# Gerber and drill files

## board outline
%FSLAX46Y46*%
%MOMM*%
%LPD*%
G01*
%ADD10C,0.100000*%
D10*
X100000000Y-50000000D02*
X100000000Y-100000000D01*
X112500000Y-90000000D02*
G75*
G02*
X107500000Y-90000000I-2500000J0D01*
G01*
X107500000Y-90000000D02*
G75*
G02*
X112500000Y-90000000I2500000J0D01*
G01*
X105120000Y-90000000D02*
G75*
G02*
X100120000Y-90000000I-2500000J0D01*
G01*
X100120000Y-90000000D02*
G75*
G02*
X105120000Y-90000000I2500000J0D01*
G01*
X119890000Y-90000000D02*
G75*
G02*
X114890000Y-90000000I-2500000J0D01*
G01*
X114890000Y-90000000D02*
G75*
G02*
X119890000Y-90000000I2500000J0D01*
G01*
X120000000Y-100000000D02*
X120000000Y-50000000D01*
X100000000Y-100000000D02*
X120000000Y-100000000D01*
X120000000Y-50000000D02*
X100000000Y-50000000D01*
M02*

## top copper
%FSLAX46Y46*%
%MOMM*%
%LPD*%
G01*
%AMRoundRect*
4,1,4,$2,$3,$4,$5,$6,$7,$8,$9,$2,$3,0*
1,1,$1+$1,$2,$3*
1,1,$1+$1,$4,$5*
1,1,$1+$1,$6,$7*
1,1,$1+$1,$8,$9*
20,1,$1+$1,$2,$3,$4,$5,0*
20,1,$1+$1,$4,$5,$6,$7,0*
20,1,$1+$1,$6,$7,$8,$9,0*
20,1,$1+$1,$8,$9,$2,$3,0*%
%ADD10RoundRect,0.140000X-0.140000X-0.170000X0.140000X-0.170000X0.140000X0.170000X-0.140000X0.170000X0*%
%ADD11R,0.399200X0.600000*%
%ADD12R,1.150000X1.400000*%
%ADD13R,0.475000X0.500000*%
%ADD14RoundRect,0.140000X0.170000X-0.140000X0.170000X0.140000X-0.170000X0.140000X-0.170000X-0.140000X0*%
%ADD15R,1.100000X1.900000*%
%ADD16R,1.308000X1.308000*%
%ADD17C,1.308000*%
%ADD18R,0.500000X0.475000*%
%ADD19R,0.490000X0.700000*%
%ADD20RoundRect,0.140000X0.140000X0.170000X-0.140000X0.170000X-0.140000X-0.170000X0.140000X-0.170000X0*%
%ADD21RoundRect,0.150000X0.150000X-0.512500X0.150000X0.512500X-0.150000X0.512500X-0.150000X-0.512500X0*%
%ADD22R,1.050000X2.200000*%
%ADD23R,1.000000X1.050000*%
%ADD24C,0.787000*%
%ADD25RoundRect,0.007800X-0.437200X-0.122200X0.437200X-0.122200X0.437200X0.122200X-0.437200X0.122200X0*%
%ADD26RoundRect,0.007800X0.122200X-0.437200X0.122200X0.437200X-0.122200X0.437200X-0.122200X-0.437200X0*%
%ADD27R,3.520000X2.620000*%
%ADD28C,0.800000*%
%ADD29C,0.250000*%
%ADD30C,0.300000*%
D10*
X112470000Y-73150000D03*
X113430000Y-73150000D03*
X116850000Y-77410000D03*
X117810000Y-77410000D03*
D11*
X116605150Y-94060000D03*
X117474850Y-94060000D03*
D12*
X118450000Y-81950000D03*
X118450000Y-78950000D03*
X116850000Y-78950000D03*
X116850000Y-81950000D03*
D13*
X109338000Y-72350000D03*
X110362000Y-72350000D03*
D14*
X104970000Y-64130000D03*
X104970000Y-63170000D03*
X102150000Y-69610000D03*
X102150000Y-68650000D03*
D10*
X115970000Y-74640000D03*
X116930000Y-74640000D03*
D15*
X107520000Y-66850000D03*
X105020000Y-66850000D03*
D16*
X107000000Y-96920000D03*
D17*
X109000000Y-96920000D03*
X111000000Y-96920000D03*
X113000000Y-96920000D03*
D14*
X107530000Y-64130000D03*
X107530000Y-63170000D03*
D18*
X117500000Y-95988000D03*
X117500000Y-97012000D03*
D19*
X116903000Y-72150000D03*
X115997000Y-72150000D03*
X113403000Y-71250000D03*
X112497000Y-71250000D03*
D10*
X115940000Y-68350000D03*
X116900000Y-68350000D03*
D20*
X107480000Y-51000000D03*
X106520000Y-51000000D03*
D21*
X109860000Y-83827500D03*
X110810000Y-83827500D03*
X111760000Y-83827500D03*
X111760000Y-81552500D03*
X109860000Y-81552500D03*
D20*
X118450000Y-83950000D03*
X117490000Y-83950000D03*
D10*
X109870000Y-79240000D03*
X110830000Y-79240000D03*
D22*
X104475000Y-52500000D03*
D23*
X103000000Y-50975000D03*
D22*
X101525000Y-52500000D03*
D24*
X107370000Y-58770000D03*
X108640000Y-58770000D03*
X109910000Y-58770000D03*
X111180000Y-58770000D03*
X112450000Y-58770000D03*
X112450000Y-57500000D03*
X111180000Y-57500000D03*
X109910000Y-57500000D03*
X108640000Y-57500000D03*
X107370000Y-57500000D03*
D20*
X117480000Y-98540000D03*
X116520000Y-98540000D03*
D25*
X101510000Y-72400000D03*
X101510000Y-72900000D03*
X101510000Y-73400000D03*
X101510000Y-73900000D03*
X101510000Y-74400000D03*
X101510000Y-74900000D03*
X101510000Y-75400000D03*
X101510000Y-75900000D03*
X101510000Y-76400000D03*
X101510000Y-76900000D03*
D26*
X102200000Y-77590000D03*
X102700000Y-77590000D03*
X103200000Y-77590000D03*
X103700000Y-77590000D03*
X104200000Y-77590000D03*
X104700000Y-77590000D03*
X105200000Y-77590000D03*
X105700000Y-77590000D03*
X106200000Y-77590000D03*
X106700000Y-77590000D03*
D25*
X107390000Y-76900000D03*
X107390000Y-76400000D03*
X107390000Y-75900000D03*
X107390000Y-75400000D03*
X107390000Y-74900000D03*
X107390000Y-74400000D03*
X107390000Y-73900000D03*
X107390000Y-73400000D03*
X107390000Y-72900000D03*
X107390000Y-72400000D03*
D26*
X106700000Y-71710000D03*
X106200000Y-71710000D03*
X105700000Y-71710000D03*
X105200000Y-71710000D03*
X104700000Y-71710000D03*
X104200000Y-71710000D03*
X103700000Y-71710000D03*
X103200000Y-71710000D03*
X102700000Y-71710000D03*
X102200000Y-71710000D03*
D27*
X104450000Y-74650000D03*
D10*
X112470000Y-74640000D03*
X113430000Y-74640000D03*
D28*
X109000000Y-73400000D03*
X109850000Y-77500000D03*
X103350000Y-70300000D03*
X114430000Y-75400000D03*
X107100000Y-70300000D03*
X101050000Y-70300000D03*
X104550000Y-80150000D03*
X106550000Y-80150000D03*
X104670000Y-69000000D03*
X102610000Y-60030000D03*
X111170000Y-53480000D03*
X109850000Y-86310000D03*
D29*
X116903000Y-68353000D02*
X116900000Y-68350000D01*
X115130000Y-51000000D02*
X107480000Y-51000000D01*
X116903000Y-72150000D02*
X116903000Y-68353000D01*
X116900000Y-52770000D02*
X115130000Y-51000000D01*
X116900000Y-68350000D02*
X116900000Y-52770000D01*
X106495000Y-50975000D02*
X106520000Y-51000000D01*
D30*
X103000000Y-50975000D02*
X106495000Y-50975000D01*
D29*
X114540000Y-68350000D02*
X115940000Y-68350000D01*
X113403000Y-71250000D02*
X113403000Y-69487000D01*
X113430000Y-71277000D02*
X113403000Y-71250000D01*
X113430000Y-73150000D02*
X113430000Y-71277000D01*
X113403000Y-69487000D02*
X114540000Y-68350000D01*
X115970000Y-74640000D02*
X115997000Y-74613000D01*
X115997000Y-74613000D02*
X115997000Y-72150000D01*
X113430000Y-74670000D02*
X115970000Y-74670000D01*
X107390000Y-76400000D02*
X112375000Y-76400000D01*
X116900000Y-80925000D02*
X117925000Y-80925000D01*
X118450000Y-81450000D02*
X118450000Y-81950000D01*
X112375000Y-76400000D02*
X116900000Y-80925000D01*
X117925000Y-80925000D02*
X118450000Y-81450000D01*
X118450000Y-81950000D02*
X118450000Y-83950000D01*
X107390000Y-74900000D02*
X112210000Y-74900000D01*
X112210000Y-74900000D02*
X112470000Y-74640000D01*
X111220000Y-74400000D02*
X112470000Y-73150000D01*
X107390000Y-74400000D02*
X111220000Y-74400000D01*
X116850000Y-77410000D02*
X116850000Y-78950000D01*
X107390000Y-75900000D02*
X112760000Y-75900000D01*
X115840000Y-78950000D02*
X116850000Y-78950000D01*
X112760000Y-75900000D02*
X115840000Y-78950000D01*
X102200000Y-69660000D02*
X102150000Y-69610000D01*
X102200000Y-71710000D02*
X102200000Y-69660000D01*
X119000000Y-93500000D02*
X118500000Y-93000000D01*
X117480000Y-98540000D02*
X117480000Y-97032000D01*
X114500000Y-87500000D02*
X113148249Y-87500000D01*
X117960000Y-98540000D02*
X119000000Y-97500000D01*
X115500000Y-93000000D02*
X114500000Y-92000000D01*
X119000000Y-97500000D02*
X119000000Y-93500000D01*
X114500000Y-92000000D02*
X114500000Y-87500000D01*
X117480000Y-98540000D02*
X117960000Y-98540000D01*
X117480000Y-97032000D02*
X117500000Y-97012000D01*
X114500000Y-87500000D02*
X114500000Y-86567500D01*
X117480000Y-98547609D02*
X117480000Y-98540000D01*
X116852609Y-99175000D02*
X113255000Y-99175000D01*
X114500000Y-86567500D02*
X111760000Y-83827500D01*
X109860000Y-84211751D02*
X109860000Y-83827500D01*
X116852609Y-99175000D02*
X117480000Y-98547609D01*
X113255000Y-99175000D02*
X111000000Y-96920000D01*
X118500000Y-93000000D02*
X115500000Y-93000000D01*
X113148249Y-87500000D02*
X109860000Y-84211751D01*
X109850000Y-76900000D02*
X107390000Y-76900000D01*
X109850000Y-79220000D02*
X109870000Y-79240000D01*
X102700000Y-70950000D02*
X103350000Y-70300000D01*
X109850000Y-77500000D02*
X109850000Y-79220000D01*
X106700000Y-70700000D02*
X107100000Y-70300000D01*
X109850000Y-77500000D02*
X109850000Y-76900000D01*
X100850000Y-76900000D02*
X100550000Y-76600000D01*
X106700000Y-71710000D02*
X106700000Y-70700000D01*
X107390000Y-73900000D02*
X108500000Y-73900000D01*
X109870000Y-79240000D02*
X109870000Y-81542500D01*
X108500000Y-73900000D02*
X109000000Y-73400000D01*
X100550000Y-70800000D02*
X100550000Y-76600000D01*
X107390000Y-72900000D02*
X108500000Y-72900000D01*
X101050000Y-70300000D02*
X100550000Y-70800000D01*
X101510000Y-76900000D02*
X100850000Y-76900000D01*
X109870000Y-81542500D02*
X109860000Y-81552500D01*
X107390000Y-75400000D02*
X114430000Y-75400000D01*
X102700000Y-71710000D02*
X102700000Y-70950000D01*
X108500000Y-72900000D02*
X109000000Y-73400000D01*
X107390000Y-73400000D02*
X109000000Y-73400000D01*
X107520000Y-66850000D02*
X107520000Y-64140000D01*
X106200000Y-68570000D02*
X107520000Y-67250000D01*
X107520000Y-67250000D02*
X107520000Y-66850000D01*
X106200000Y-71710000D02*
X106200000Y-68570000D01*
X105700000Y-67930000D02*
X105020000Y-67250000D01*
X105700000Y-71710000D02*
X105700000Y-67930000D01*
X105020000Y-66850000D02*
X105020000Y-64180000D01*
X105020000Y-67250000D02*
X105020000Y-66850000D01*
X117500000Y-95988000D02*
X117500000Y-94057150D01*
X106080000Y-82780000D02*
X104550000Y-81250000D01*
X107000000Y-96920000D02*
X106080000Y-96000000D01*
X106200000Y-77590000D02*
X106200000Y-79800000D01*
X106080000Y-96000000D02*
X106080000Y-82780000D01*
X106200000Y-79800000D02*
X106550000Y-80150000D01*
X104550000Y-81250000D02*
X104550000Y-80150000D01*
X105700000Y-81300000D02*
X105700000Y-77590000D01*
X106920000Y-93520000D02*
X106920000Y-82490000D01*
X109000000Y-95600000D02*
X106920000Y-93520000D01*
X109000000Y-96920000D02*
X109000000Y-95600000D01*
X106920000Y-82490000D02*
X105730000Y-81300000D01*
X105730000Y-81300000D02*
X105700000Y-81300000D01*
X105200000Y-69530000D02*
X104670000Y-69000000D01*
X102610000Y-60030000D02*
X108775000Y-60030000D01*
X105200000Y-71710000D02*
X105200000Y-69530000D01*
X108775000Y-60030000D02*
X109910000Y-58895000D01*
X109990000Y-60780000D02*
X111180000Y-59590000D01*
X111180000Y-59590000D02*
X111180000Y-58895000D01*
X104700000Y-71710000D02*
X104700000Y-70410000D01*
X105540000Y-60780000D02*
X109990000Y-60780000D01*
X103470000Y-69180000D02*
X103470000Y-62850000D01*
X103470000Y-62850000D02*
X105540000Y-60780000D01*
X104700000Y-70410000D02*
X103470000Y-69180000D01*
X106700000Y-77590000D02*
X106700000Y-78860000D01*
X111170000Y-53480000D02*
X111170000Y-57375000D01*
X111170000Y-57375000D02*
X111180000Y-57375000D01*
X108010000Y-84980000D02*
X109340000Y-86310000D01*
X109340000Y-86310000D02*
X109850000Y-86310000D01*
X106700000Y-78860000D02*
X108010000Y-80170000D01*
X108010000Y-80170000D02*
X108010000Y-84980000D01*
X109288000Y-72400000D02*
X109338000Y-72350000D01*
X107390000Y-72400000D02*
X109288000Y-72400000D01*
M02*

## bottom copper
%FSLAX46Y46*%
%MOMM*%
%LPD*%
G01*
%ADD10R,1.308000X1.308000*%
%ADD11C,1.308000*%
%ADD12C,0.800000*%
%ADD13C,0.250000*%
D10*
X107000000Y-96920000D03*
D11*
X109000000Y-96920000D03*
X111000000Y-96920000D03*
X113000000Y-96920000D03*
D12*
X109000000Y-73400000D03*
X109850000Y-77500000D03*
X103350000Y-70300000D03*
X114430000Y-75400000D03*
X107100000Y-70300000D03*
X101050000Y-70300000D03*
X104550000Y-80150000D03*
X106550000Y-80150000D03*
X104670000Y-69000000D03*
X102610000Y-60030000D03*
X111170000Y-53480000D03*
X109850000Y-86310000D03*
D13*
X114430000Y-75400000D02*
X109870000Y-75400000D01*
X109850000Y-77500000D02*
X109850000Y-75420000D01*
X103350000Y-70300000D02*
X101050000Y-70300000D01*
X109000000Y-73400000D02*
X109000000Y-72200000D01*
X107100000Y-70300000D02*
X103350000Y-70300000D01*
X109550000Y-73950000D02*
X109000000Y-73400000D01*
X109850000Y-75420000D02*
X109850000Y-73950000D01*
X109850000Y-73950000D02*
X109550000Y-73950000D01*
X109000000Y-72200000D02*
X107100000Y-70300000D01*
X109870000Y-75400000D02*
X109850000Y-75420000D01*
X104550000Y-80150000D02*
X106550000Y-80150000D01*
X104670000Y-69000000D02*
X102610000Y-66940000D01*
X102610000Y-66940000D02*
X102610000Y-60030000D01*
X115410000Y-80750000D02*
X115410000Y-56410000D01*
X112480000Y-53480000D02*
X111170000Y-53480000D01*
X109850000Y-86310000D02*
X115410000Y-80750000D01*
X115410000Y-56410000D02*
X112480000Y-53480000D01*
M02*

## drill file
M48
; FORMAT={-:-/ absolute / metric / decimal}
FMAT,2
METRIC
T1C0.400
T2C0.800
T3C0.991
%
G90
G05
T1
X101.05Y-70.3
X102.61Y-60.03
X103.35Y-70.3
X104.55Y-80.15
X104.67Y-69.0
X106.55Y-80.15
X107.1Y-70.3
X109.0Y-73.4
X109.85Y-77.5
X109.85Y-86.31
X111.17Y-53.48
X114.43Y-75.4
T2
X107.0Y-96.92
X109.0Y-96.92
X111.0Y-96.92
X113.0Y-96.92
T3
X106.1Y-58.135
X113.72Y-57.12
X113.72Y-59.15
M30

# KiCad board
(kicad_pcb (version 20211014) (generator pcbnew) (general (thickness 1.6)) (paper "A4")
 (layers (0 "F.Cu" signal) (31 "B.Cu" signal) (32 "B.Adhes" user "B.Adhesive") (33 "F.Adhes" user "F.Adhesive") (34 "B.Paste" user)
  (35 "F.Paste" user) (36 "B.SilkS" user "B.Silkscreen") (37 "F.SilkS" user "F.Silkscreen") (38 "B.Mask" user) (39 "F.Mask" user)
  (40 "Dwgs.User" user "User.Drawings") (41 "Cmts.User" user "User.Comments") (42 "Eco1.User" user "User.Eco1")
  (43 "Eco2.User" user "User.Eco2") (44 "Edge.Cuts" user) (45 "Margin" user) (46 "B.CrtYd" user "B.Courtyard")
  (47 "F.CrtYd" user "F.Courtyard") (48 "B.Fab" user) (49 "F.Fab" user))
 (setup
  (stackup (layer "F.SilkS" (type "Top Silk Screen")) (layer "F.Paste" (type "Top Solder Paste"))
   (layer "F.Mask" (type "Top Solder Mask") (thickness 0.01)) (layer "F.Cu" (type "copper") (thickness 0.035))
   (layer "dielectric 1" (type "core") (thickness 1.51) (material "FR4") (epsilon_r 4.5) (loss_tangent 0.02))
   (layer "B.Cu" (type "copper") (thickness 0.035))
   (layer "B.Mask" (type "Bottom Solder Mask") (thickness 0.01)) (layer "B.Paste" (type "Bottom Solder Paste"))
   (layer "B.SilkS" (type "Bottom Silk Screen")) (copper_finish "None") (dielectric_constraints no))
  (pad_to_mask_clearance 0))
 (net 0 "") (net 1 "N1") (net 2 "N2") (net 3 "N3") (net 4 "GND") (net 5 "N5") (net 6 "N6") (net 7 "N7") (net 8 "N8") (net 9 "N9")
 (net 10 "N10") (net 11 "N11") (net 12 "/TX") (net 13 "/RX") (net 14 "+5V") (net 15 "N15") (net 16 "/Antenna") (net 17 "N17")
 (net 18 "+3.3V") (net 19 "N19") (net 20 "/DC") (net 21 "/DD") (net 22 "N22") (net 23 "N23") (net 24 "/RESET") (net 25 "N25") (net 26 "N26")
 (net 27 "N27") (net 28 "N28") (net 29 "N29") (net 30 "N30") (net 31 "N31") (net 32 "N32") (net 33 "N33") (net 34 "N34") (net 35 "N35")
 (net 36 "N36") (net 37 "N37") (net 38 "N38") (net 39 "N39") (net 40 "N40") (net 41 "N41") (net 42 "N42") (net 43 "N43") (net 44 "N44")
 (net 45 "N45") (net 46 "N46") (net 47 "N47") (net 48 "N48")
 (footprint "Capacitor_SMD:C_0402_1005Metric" (layer "F.Cu") (at 112.95 73.15)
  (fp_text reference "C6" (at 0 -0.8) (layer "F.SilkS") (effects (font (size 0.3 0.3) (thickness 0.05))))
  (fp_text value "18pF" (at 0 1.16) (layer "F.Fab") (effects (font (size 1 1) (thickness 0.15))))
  (pad "1" smd roundrect (at -0.48 0) (size 0.56 0.62) (layers "F.Cu" "F.Paste" "F.Mask") (roundrect_rratio 0.25) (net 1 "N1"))
  (pad "2" smd roundrect (at 0.48 0) (size 0.56 0.62) (layers "F.Cu" "F.Paste" "F.Mask") (roundrect_rratio 0.25) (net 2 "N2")))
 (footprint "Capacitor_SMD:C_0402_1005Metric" (layer "F.Cu") (at 117.33 77.41)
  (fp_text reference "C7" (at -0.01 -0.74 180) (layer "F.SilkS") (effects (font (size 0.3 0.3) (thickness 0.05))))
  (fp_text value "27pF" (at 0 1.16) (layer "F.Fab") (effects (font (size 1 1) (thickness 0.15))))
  (pad "1" smd roundrect (at -0.48 0) (size 0.56 0.62) (layers "F.Cu" "F.Paste" "F.Mask") (roundrect_rratio 0.25) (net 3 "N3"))
  (pad "2" smd roundrect (at 0.48 0) (size 0.56 0.62) (layers "F.Cu" "F.Paste" "F.Mask") (roundrect_rratio 0.25) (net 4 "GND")))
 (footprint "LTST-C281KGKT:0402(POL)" (layer "F.Cu") (at 117.04 94.06)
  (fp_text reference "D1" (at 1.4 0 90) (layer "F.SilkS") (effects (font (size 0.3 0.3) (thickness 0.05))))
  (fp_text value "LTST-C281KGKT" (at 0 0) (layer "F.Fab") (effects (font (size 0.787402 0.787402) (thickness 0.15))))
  (pad "1" smd rect locked (at -0.43485 0) (size 0.3992 0.6) (layers "F.Cu" "F.Paste" "F.Mask") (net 4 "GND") (solder_mask_margin 0.102))
  (pad "2" smd rect locked (at 0.43485 0) (size 0.3992 0.6) (layers "F.Cu" "F.Paste" "F.Mask") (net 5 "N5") (solder_mask_margin 0.102)))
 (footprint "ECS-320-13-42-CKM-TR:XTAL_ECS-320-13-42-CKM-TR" (layer "F.Cu") (at 117.65 80.45 90)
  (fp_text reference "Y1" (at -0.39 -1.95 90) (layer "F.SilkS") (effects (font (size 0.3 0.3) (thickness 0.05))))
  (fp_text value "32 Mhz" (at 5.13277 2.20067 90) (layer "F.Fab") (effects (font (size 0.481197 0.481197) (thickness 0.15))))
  (pad "1" smd rect locked (at -1.5 0.8) (size 1.15 1.4) (layers "F.Cu" "F.Paste" "F.Mask") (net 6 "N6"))
  (pad "2" smd rect locked (at 1.5 0.8) (size 1.15 1.4) (layers "F.Cu" "F.Paste" "F.Mask") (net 4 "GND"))
  (pad "3" smd rect locked (at 1.5 -0.8) (size 1.15 1.4) (layers "F.Cu" "F.Paste" "F.Mask") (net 3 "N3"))
  (pad "4" smd rect locked (at -1.5 -0.8) (size 1.15 1.4) (layers "F.Cu" "F.Paste" "F.Mask") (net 4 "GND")))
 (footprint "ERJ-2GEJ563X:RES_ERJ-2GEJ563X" (layer "F.Cu") (at 109.85 72.35)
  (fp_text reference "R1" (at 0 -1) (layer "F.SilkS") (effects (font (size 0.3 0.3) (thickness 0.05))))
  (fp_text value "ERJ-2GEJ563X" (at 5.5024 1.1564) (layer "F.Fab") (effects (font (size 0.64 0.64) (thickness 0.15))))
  (pad "1" smd rect locked (at -0.512 0) (size 0.475 0.5) (layers "F.Cu" "F.Paste" "F.Mask") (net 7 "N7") (solder_mask_margin 0.102))
  (pad "2" smd rect locked (at 0.512 0) (size 0.475 0.5) (layers "F.Cu" "F.Paste" "F.Mask") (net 4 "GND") (solder_mask_margin 0.102)))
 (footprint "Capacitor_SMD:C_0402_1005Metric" (layer "F.Cu") (at 104.97 63.65 90)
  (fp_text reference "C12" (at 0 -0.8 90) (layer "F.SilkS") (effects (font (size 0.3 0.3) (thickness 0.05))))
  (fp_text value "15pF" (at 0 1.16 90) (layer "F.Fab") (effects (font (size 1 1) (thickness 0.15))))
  (pad "1" smd roundrect (at -0.48 0 90) (size 0.56 0.62) (layers "F.Cu" "F.Paste" "F.Mask") (roundrect_rratio 0.25) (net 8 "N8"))
  (pad "2" smd roundrect (at 0.48 0 90) (size 0.56 0.62) (layers "F.Cu" "F.Paste" "F.Mask") (roundrect_rratio 0.25) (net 4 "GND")))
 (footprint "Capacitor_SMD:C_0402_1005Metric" (layer "F.Cu") (at 102.15 69.13 90)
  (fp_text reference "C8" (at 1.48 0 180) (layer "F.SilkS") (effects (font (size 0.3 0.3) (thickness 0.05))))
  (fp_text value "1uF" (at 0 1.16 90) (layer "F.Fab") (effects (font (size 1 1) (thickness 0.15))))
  (pad "1" smd roundrect (at -0.48 0 90) (size 0.56 0.62) (layers "F.Cu" "F.Paste" "F.Mask") (roundrect_rratio 0.25) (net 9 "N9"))
  (pad "2" smd roundrect (at 0.48 0 90) (size 0.56 0.62) (layers "F.Cu" "F.Paste" "F.Mask") (roundrect_rratio 0.25) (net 4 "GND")))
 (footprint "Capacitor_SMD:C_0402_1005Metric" (layer "F.Cu") (at 116.45 74.64)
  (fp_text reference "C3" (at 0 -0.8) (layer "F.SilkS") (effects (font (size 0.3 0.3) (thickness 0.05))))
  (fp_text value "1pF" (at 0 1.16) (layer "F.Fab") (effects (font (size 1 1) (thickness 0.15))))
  (pad "1" smd roundrect (at -0.48 0) (size 0.56 0.62) (layers "F.Cu" "F.Paste" "F.Mask") (roundrect_rratio 0.25) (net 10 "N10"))
  (pad "2" smd roundrect (at 0.48 0) (size 0.56 0.62) (layers "F.Cu" "F.Paste" "F.Mask") (roundrect_rratio 0.25) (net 4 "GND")))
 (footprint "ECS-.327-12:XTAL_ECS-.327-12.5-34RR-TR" (layer "F.Cu") (at 106.27 66.85 180)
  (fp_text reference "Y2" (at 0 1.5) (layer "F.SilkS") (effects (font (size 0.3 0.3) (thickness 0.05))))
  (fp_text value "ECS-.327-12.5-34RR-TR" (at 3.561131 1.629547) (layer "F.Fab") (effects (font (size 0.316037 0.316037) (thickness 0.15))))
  (pad "1" smd rect locked (at -1.25 0 180) (size 1.1 1.9) (layers "F.Cu" "F.Paste" "F.Mask") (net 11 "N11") (solder_mask_margin 0.102))
  (pad "2" smd rect locked (at 1.25 0 180) (size 1.1 1.9) (layers "F.Cu" "F.Paste" "F.Mask") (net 8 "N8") (solder_mask_margin 0.102)))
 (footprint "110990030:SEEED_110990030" (layer "F.Cu") (at 110 96.92)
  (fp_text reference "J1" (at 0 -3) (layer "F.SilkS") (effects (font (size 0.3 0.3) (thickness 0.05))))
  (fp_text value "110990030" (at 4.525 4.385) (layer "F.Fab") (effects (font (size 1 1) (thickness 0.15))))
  (pad "1" thru_hole rect locked (at -3 0) (size 1.308 1.308) (drill 0.8) (layers *.Cu *.Mask) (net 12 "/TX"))
  (pad "2" thru_hole circle locked (at -1 0) (size 1.308 1.308) (drill 0.8) (layers *.Cu *.Mask) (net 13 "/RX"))
  (pad "3" thru_hole circle locked (at 1 0) (size 1.308 1.308) (drill 0.8) (layers *.Cu *.Mask) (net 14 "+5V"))
  (pad "4" thru_hole circle locked (at 3 0) (size 1.308 1.308) (drill 0.8) (layers *.Cu *.Mask) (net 4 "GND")))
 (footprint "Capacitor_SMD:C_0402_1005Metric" (layer "F.Cu") (at 107.53 63.65 90)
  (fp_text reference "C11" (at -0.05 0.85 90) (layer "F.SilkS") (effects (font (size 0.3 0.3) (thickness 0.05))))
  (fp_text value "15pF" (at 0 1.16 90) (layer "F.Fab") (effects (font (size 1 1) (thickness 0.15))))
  (pad "1" smd roundrect (at -0.48 0 90) (size 0.56 0.62) (layers "F.Cu" "F.Paste" "F.Mask") (roundrect_rratio 0.25) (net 11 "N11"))
  (pad "2" smd roundrect (at 0.48 0 90) (size 0.56 0.62) (layers "F.Cu" "F.Paste" "F.Mask") (roundrect_rratio 0.25) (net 4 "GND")))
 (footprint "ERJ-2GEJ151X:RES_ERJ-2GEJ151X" (layer "F.Cu") (at 117.5 96.5 -90)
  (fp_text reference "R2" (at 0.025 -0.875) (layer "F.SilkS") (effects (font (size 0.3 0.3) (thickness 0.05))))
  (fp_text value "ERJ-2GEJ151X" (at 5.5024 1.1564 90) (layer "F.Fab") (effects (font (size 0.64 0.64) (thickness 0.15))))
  (pad "1" smd rect locked (at -0.512 0 270) (size 0.475 0.5) (layers "F.Cu" "F.Paste" "F.Mask") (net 5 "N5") (solder_mask_margin 0.102))
  (pad "2" smd rect locked (at 0.512 0 270) (size 0.475 0.5) (layers "F.Cu" "F.Paste" "F.Mask") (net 14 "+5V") (solder_mask_margin 0.102)))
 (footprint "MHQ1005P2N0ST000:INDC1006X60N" (layer "F.Cu") (at 116.45 72.15 180)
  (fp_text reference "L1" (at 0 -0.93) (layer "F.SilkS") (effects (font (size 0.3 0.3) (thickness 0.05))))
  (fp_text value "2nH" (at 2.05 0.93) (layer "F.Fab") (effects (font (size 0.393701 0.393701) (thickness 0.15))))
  (pad "1" smd rect locked (at -0.453 0 180) (size 0.49 0.7) (layers "F.Cu" "F.Paste" "F.Mask") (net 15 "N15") (solder_mask_margin 0.102))
  (pad "2" smd rect locked (at 0.453 0 180) (size 0.49 0.7) (layers "F.Cu" "F.Paste" "F.Mask") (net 10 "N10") (solder_mask_margin 0.102)))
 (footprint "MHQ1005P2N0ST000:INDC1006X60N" (layer "F.Cu") (at 112.95 71.25 180)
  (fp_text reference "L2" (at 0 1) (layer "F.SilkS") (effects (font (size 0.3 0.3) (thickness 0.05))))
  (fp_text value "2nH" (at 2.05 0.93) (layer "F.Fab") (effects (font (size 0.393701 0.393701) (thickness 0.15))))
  (pad "1" smd rect locked (at -0.453 0 180) (size 0.49 0.7) (layers "F.Cu" "F.Paste" "F.Mask") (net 2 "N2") (solder_mask_margin 0.102))
  (pad "2" smd rect locked (at 0.453 0 180) (size 0.49 0.7) (layers "F.Cu" "F.Paste" "F.Mask") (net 4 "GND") (solder_mask_margin 0.102)))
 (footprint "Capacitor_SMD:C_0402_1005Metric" (layer "F.Cu") (at 116.42 68.35)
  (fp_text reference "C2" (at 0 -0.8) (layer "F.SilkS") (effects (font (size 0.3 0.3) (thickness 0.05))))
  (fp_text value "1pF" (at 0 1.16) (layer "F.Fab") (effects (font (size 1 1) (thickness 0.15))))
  (pad "1" smd roundrect (at -0.48 0) (size 0.56 0.62) (layers "F.Cu" "F.Paste" "F.Mask") (roundrect_rratio 0.25) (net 2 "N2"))
  (pad "2" smd roundrect (at 0.48 0) (size 0.56 0.62) (layers "F.Cu" "F.Paste" "F.Mask") (roundrect_rratio 0.25) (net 15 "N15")))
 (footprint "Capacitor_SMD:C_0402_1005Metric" (layer "F.Cu") (at 107 51 180)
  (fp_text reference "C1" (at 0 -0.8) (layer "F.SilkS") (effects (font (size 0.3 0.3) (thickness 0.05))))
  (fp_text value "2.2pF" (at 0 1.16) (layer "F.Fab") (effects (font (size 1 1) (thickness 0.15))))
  (pad "1" smd roundrect (at -0.48 0 180) (size 0.56 0.62) (layers "F.Cu" "F.Paste" "F.Mask") (roundrect_rratio 0.25) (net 15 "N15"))
  (pad "2" smd roundrect (at 0.48 0 180) (size 0.56 0.62) (layers "F.Cu" "F.Paste" "F.Mask") (roundrect_rratio 0.25) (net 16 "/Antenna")))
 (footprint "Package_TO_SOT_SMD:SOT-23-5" (layer "F.Cu") (at 110.81 82.69 90)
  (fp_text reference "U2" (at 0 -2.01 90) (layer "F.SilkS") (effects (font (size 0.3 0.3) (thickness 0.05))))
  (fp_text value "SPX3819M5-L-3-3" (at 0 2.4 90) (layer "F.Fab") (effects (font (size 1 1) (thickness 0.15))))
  (pad "1" smd roundrect (at -1.1375 -0.95 90) (size 1.325 0.6) (layers "F.Cu" "F.Paste" "F.Mask") (roundrect_rratio 0.25) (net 14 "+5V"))
  (pad "2" smd roundrect (at -1.1375 0 90) (size 1.325 0.6) (layers "F.Cu" "F.Paste" "F.Mask") (roundrect_rratio 0.25) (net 4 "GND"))
  (pad "3" smd roundrect (at -1.1375 0.95 90) (size 1.325 0.6) (layers "F.Cu" "F.Paste" "F.Mask") (roundrect_rratio 0.25) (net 14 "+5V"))
  (pad "4" smd roundrect (at 1.1375 0.95 90) (size 1.325 0.6) (layers "F.Cu" "F.Paste" "F.Mask") (roundrect_rratio 0.25) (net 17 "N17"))
  (pad "5" smd roundrect (at 1.1375 -0.95 90) (size 1.325 0.6) (layers "F.Cu" "F.Paste" "F.Mask") (roundrect_rratio 0.25) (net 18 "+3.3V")))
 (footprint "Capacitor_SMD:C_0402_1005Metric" (layer "F.Cu") (at 117.97 83.95 180)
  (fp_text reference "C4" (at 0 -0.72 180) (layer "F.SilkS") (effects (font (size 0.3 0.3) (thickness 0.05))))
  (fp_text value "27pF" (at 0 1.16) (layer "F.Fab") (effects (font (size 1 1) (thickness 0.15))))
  (pad "1" smd roundrect (at -0.48 0 180) (size 0.56 0.62) (layers "F.Cu" "F.Paste" "F.Mask") (roundrect_rratio 0.25) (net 6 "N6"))
  (pad "2" smd roundrect (at 0.48 0 180) (size 0.56 0.62) (layers "F.Cu" "F.Paste" "F.Mask") (roundrect_rratio 0.25) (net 4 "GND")))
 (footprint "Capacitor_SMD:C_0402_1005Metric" (layer "F.Cu") (at 110.35 79.24)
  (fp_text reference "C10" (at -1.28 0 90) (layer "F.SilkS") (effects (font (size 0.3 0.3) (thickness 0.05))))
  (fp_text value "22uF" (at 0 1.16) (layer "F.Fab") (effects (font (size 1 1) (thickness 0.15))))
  (pad "1" smd roundrect (at -0.48 0) (size 0.56 0.62) (layers "F.Cu" "F.Paste" "F.Mask") (roundrect_rratio 0.25) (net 18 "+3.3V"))
  (pad "2" smd roundrect (at 0.48 0) (size 0.56 0.62) (layers "F.Cu" "F.Paste" "F.Mask") (roundrect_rratio 0.25) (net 4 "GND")))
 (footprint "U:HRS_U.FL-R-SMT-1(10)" (layer "F.Cu") (at 103 52.5 180)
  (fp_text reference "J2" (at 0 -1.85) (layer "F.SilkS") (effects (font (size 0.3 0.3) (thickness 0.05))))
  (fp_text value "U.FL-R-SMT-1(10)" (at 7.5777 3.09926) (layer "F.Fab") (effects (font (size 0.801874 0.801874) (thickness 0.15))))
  (pad "1" smd rect locked (at -1.475 0 180) (size 1.05 2.2) (layers "F.Cu" "F.Paste" "F.Mask") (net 4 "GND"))
  (pad "2" smd rect locked (at 0 1.525 180) (size 1 1.05) (layers "F.Cu" "F.Paste" "F.Mask") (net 16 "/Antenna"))
  (pad "3" smd rect locked (at 1.475 0 180) (size 1.05 2.2) (layers "F.Cu" "F.Paste" "F.Mask") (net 4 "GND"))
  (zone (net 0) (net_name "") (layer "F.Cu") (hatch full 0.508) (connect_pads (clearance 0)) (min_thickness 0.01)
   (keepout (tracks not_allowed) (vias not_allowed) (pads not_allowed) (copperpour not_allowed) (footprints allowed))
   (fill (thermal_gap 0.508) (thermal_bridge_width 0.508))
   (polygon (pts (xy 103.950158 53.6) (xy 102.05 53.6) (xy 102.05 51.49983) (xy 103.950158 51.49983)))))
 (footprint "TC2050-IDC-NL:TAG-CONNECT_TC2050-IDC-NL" (layer "F.Cu") (at 107.37 58.77 90)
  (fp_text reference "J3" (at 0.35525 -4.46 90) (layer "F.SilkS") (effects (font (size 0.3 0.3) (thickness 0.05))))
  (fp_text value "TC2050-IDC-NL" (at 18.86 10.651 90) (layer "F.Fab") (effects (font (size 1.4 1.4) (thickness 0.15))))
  (pad "" np_thru_hole circle locked (at -0.38 6.35 90) (size 0.991 0.991) (drill 0.991) (layers *.Cu *.Mask))
  (pad "" np_thru_hole circle locked (at 0.635 -1.27 90) (size 0.991 0.991) (drill 0.991) (layers *.Cu *.Mask))
  (pad "" np_thru_hole circle locked (at 1.65 6.35 90) (size 0.991 0.991) (drill 0.991) (layers *.Cu *.Mask))
  (pad "1" smd circle locked (at 0 0) (size 0.787 0.787) (layers "F.Cu" "F.Mask") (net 4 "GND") (solder_mask_margin 0.102))
  (pad "2" smd circle locked (at 0 1.27) (size 0.787 0.787) (layers "F.Cu" "F.Mask") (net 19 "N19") (solder_mask_margin 0.102))
  (pad "3" smd circle locked (at 0 2.54) (size 0.787 0.787) (layers "F.Cu" "F.Mask") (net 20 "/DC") (solder_mask_margin 0.102))
  (pad "4" smd circle locked (at 0 3.81) (size 0.787 0.787) (layers "F.Cu" "F.Mask") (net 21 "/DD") (solder_mask_margin 0.102))
  (pad "5" smd circle locked (at 0 5.08) (size 0.787 0.787) (layers "F.Cu" "F.Mask") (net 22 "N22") (solder_mask_margin 0.102))
  (pad "6" smd circle locked (at 1.27 5.08 180) (size 0.787 0.787) (layers "F.Cu" "F.Mask") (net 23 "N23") (solder_mask_margin 0.102))
  (pad "7" smd circle locked (at 1.27 3.81 180) (size 0.787 0.787) (layers "F.Cu" "F.Mask") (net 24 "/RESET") (solder_mask_margin 0.102))
  (pad "8" smd circle locked (at 1.27 2.54 180) (size 0.787 0.787) (layers "F.Cu" "F.Mask") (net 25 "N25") (solder_mask_margin 0.102))
  (pad "9" smd circle locked (at 1.27 1.27 180) (size 0.787 0.787) (layers "F.Cu" "F.Mask") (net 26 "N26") (solder_mask_margin 0.102))
  (pad "10" smd circle locked (at 1.27 0 180) (size 0.787 0.787) (layers "F.Cu" "F.Mask") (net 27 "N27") (solder_mask_margin 0.102))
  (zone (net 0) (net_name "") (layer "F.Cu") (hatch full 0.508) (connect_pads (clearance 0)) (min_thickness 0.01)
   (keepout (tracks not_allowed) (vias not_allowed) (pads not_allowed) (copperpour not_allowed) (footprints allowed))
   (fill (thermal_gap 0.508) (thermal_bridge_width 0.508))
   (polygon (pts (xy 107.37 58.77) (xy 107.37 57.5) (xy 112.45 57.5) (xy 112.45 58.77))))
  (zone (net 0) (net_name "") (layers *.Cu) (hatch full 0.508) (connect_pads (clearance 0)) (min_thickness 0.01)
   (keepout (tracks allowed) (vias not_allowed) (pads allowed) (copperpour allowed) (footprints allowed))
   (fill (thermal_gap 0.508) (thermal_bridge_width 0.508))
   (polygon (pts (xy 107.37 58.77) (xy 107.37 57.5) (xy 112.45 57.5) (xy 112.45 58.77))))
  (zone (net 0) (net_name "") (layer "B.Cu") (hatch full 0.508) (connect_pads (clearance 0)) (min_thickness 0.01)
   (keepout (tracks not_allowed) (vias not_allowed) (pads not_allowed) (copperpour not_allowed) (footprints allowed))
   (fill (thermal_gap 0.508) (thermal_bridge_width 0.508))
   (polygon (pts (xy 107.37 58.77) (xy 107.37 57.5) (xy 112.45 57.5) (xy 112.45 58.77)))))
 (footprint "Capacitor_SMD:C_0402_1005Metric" (layer "F.Cu") (at 117 98.54 180)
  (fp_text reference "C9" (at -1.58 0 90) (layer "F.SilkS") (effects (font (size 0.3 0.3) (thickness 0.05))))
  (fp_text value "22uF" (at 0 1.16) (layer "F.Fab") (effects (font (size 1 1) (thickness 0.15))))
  (pad "1" smd roundrect (at -0.48 0 180) (size 0.56 0.62) (layers "F.Cu" "F.Paste" "F.Mask") (roundrect_rratio 0.25) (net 14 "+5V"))
  (pad "2" smd roundrect (at 0.48 0 180) (size 0.56 0.62) (layers "F.Cu" "F.Paste" "F.Mask") (roundrect_rratio 0.25) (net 4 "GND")))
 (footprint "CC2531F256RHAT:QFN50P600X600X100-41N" (layer "F.Cu") (at 104.45 74.65)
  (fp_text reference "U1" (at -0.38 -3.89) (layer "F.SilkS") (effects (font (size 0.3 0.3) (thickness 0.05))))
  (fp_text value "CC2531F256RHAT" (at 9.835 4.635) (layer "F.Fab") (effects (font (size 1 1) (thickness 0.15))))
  (pad "1" smd roundrect locked (at -2.94 -2.25) (size 0.89 0.26) (layers "F.Cu" "F.Paste" "F.Mask") (roundrect_rratio 0.03) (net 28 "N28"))
  (pad "2" smd roundrect locked (at -2.94 -1.75) (size 0.89 0.26) (layers "F.Cu" "F.Paste" "F.Mask") (roundrect_rratio 0.03) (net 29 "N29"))
  (pad "3" smd roundrect locked (at -2.94 -1.25) (size 0.89 0.26) (layers "F.Cu" "F.Paste" "F.Mask") (roundrect_rratio 0.03) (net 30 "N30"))
  (pad "4" smd roundrect locked (at -2.94 -0.75) (size 0.89 0.26) (layers "F.Cu" "F.Paste" "F.Mask") (roundrect_rratio 0.03) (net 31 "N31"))
  (pad "5" smd roundrect locked (at -2.94 -0.25) (size 0.89 0.26) (layers "F.Cu" "F.Paste" "F.Mask") (roundrect_rratio 0.03) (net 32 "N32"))
  (pad "6" smd roundrect locked (at -2.94 0.25) (size 0.89 0.26) (layers "F.Cu" "F.Paste" "F.Mask") (roundrect_rratio 0.03) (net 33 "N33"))
  (pad "7" smd roundrect locked (at -2.94 0.75) (size 0.89 0.26) (layers "F.Cu" "F.Paste" "F.Mask") (roundrect_rratio 0.03) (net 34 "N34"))
  (pad "8" smd roundrect locked (at -2.94 1.25) (size 0.89 0.26) (layers "F.Cu" "F.Paste" "F.Mask") (roundrect_rratio 0.03) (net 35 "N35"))
  (pad "9" smd roundrect locked (at -2.94 1.75) (size 0.89 0.26) (layers "F.Cu" "F.Paste" "F.Mask") (roundrect_rratio 0.03) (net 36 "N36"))
  (pad "10" smd roundrect locked (at -2.94 2.25) (size 0.89 0.26) (layers "F.Cu" "F.Paste" "F.Mask") (roundrect_rratio 0.03)
   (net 18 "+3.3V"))
  (pad "11" smd roundrect locked (at -2.25 2.94 90) (size 0.89 0.26) (layers "F.Cu" "F.Paste" "F.Mask") (roundrect_rratio 0.03)
   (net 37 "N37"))
  (pad "12" smd roundrect locked (at -1.75 2.94 90) (size 0.89 0.26) (layers "F.Cu" "F.Paste" "F.Mask") (roundrect_rratio 0.03)
   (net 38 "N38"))
  (pad "13" smd roundrect locked (at -1.25 2.94 90) (size 0.89 0.26) (layers "F.Cu" "F.Paste" "F.Mask") (roundrect_rratio 0.03)
   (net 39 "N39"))
  (pad "14" smd roundrect locked (at -0.75 2.94 90) (size 0.89 0.26) (layers "F.Cu" "F.Paste" "F.Mask") (roundrect_rratio 0.03)
   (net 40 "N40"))
  (pad "15" smd roundrect locked (at -0.25 2.94 90) (size 0.89 0.26) (layers "F.Cu" "F.Paste" "F.Mask") (roundrect_rratio 0.03)
   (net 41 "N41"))
  (pad "16" smd roundrect locked (at 0.25 2.94 90) (size 0.89 0.26) (layers "F.Cu" "F.Paste" "F.Mask") (roundrect_rratio 0.03)
   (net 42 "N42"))
  (pad "17" smd roundrect locked (at 0.75 2.94 90) (size 0.89 0.26) (layers "F.Cu" "F.Paste" "F.Mask") (roundrect_rratio 0.03)
   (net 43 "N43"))
  (pad "18" smd roundrect locked (at 1.25 2.94 90) (size 0.89 0.26) (layers "F.Cu" "F.Paste" "F.Mask") (roundrect_rratio 0.03)
   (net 13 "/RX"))
  (pad "19" smd roundrect locked (at 1.75 2.94 90) (size 0.89 0.26) (layers "F.Cu" "F.Paste" "F.Mask") (roundrect_rratio 0.03)
   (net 12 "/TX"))
  (pad "20" smd roundrect locked (at 2.25 2.94 90) (size 0.89 0.26) (layers "F.Cu" "F.Paste" "F.Mask") (roundrect_rratio 0.03)
   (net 24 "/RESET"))
  (pad "21" smd roundrect locked (at 2.94 2.25) (size 0.89 0.26) (layers "F.Cu" "F.Paste" "F.Mask") (roundrect_rratio 0.03) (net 18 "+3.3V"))
  (pad "22" smd roundrect locked (at 2.94 1.75) (size 0.89 0.26) (layers "F.Cu" "F.Paste" "F.Mask") (roundrect_rratio 0.03) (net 6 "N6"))
  (pad "23" smd roundrect locked (at 2.94 1.25) (size 0.89 0.26) (layers "F.Cu" "F.Paste" "F.Mask") (roundrect_rratio 0.03) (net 3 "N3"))
  (pad "24" smd roundrect locked (at 2.94 0.75) (size 0.89 0.26) (layers "F.Cu" "F.Paste" "F.Mask") (roundrect_rratio 0.03) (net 18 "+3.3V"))
  (pad "25" smd roundrect locked (at 2.94 0.25) (size 0.89 0.26) (layers "F.Cu" "F.Paste" "F.Mask") (roundrect_rratio 0.03) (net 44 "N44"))
  (pad "26" smd roundrect locked (at 2.94 -0.25) (size 0.89 0.26) (layers "F.Cu" "F.Paste" "F.Mask") (roundrect_rratio 0.03) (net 1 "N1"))
  (pad "27" smd roundrect locked (at 2.94 -0.75) (size 0.89 0.26) (layers "F.Cu" "F.Paste" "F.Mask") (roundrect_rratio 0.03)
   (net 18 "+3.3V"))
  (pad "28" smd roundrect locked (at 2.94 -1.25) (size 0.89 0.26) (layers "F.Cu" "F.Paste" "F.Mask") (roundrect_rratio 0.03)
   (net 18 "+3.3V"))
  (pad "29" smd roundrect locked (at 2.94 -1.75) (size 0.89 0.26) (layers "F.Cu" "F.Paste" "F.Mask") (roundrect_rratio 0.03)
   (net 18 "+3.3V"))
  (pad "30" smd roundrect locked (at 2.94 -2.25) (size 0.89 0.26) (layers "F.Cu" "F.Paste" "F.Mask") (roundrect_rratio 0.03) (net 7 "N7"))
  (pad "31" smd roundrect locked (at 2.25 -2.94 90) (size 0.89 0.26) (layers "F.Cu" "F.Paste" "F.Mask") (roundrect_rratio 0.03)
   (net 18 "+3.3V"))
  (pad "32" smd roundrect locked (at 1.75 -2.94 90) (size 0.89 0.26) (layers "F.Cu" "F.Paste" "F.Mask") (roundrect_rratio 0.03)
   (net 11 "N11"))
  (pad "33" smd roundrect locked (at 1.25 -2.94 90) (size 0.89 0.26) (layers "F.Cu" "F.Paste" "F.Mask") (roundrect_rratio 0.03) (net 8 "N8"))
  (pad "34" smd roundrect locked (at 0.75 -2.94 90) (size 0.89 0.26) (layers "F.Cu" "F.Paste" "F.Mask") (roundrect_rratio 0.03)
   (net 20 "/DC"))
  (pad "35" smd roundrect locked (at 0.25 -2.94 90) (size 0.89 0.26) (layers "F.Cu" "F.Paste" "F.Mask") (roundrect_rratio 0.03)
   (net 21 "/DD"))
  (pad "36" smd roundrect locked (at -0.25 -2.94 90) (size 0.89 0.26) (layers "F.Cu" "F.Paste" "F.Mask") (roundrect_rratio 0.03)
   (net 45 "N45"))
  (pad "37" smd roundrect locked (at -0.75 -2.94 90) (size 0.89 0.26) (layers "F.Cu" "F.Paste" "F.Mask") (roundrect_rratio 0.03)
   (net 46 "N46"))
  (pad "38" smd roundrect locked (at -1.25 -2.94 90) (size 0.89 0.26) (layers "F.Cu" "F.Paste" "F.Mask") (roundrect_rratio 0.03)
   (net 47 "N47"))
  (pad "39" smd roundrect locked (at -1.75 -2.94 90) (size 0.89 0.26) (layers "F.Cu" "F.Paste" "F.Mask") (roundrect_rratio 0.03)
   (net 18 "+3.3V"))
  (pad "40" smd roundrect locked (at -2.25 -2.94 90) (size 0.89 0.26) (layers "F.Cu" "F.Paste" "F.Mask") (roundrect_rratio 0.03)
   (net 9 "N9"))
  (pad "41" smd rect locked (at 0 0) (size 3.52 2.62) (layers "F.Cu" "F.Mask") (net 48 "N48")))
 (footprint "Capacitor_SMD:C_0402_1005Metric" (layer "F.Cu") (at 112.95 74.64)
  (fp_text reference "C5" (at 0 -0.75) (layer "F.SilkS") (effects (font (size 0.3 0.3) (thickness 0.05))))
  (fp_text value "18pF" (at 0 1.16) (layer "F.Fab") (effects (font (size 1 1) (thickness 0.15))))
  (pad "1" smd roundrect (at -0.48 0) (size 0.56 0.62) (layers "F.Cu" "F.Paste" "F.Mask") (roundrect_rratio 0.25) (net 44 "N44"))
  (pad "2" smd roundrect (at 0.48 0) (size 0.56 0.62) (layers "F.Cu" "F.Paste" "F.Mask") (roundrect_rratio 0.25) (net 10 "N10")))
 (gr_line (start 100 50) (end 100 100) (layer "Edge.Cuts") (width 0.1))
 (gr_circle (center 110 90) (end 112.5 90) (layer "Edge.Cuts") (width 0.1) (fill none))
 (gr_circle (center 102.62 90) (end 105.12 90) (layer "Edge.Cuts") (width 0.1) (fill none))
 (gr_circle (center 117.39 90) (end 114.89 90) (layer "Edge.Cuts") (width 0.1) (fill none))
 (gr_line (start 120 100) (end 120 50) (layer "Edge.Cuts") (width 0.1))
 (gr_line (start 100 100) (end 120 100) (layer "Edge.Cuts") (width 0.1))
 (gr_line (start 120 50) (end 100 50) (layer "Edge.Cuts") (width 0.1))
 (segment (start 116.903 68.353) (end 116.9 68.35) (width 0.25) (layer "F.Cu") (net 15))
 (segment (start 115.13 51) (end 107.48 51) (width 0.25) (layer "F.Cu") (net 15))
 (segment (start 116.903 72.15) (end 116.903 68.353) (width 0.25) (layer "F.Cu") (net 15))
 (segment (start 116.9 52.77) (end 115.13 51) (width 0.25) (layer "F.Cu") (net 15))
 (segment (start 116.9 68.35) (end 116.9 52.77) (width 0.25) (layer "F.Cu") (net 15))
 (segment (start 106.495 50.975) (end 106.52 51) (width 0.25) (layer "F.Cu") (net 16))
 (segment (start 103 50.975) (end 106.495 50.975) (width 0.3) (layer "F.Cu") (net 16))
 (segment (start 114.54 68.35) (end 115.94 68.35) (width 0.25) (layer "F.Cu") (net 2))
 (segment (start 113.403 71.25) (end 113.403 69.487) (width 0.25) (layer "F.Cu") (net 2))
 (segment (start 113.43 71.277) (end 113.403 71.25) (width 0.25) (layer "F.Cu") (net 2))
 (segment (start 113.43 73.15) (end 113.43 71.277) (width 0.25) (layer "F.Cu") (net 2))
 (segment (start 113.403 69.487) (end 114.54 68.35) (width 0.25) (layer "F.Cu") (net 2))
 (segment (start 115.97 74.64) (end 115.997 74.613) (width 0.25) (layer "F.Cu") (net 10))
 (segment (start 115.997 74.613) (end 115.997 72.15) (width 0.25) (layer "F.Cu") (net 10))
 (segment (start 113.43 74.67) (end 115.97 74.67) (width 0.25) (layer "F.Cu") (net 10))
 (segment (start 107.39 76.4) (end 112.375 76.4) (width 0.25) (layer "F.Cu") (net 6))
 (segment (start 116.9 80.925) (end 117.925 80.925) (width 0.25) (layer "F.Cu") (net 6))
 (segment (start 118.45 81.45) (end 118.45 81.95) (width 0.25) (layer "F.Cu") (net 6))
 (segment (start 112.375 76.4) (end 116.9 80.925) (width 0.25) (layer "F.Cu") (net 6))
 (segment (start 117.925 80.925) (end 118.45 81.45) (width 0.25) (layer "F.Cu") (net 6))
 (segment (start 118.45 81.95) (end 118.45 83.95) (width 0.25) (layer "F.Cu") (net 6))
 (segment (start 107.39 74.9) (end 112.21 74.9) (width 0.25) (layer "F.Cu") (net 44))
 (segment (start 112.21 74.9) (end 112.47 74.64) (width 0.25) (layer "F.Cu") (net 44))
 (segment (start 111.22 74.4) (end 112.47 73.15) (width 0.25) (layer "F.Cu") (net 1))
 (segment (start 107.39 74.4) (end 111.22 74.4) (width 0.25) (layer "F.Cu") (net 1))
 (segment (start 116.85 77.41) (end 116.85 78.95) (width 0.25) (layer "F.Cu") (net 3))
 (segment (start 107.39 75.9) (end 112.76 75.9) (width 0.25) (layer "F.Cu") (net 3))
 (segment (start 115.84 78.95) (end 116.85 78.95) (width 0.25) (layer "F.Cu") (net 3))
 (segment (start 112.76 75.9) (end 115.84 78.95) (width 0.25) (layer "F.Cu") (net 3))
 (segment (start 102.2 69.66) (end 102.15 69.61) (width 0.25) (layer "F.Cu") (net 9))
 (segment (start 102.2 71.71) (end 102.2 69.66) (width 0.25) (layer "F.Cu") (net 9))
 (segment (start 119 93.5) (end 118.5 93) (width 0.25) (layer "F.Cu") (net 14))
 (segment (start 117.48 98.54) (end 117.48 97.032) (width 0.25) (layer "F.Cu") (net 14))
 (segment (start 114.5 87.5) (end 113.148249 87.5) (width 0.25) (layer "F.Cu") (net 14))
 (segment (start 117.96 98.54) (end 119 97.5) (width 0.25) (layer "F.Cu") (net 14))
 (segment (start 115.5 93) (end 114.5 92) (width 0.25) (layer "F.Cu") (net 14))
 (segment (start 119 97.5) (end 119 93.5) (width 0.25) (layer "F.Cu") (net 14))
 (segment (start 114.5 92) (end 114.5 87.5) (width 0.25) (layer "F.Cu") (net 14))
 (segment (start 117.48 98.54) (end 117.96 98.54) (width 0.25) (layer "F.Cu") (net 14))
 (segment (start 117.48 97.032) (end 117.5 97.012) (width 0.25) (layer "F.Cu") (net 14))
 (segment (start 114.5 87.5) (end 114.5 86.5675) (width 0.25) (layer "F.Cu") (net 14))
 (segment (start 117.48 98.547609) (end 117.48 98.54) (width 0.25) (layer "F.Cu") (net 14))
 (segment (start 116.852609 99.175) (end 113.255 99.175) (width 0.25) (layer "F.Cu") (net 14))
 (segment (start 114.5 86.5675) (end 111.76 83.8275) (width 0.25) (layer "F.Cu") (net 14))
 (segment (start 109.86 84.211751) (end 109.86 83.8275) (width 0.25) (layer "F.Cu") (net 14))
 (segment (start 116.852609 99.175) (end 117.48 98.547609) (width 0.25) (layer "F.Cu") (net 14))
 (segment (start 113.255 99.175) (end 111 96.92) (width 0.25) (layer "F.Cu") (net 14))
 (segment (start 118.5 93) (end 115.5 93) (width 0.25) (layer "F.Cu") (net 14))
 (segment (start 113.148249 87.5) (end 109.86 84.211751) (width 0.25) (layer "F.Cu") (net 14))
 (segment (start 109.85 76.9) (end 107.39 76.9) (width 0.25) (layer "F.Cu") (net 18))
 (segment (start 109.85 79.22) (end 109.87 79.24) (width 0.25) (layer "F.Cu") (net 18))
 (segment (start 102.7 70.95) (end 103.35 70.3) (width 0.25) (layer "F.Cu") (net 18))
 (segment (start 109.85 77.5) (end 109.85 79.22) (width 0.25) (layer "F.Cu") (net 18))
 (segment (start 106.7 70.7) (end 107.1 70.3) (width 0.25) (layer "F.Cu") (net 18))
 (segment (start 109.85 77.5) (end 109.85 76.9) (width 0.25) (layer "F.Cu") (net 18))
 (segment (start 100.85 76.9) (end 100.55 76.6) (width 0.25) (layer "F.Cu") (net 18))
 (segment (start 106.7 71.71) (end 106.7 70.7) (width 0.25) (layer "F.Cu") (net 18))
 (segment (start 107.39 73.9) (end 108.5 73.9) (width 0.25) (layer "F.Cu") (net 18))
 (segment (start 109.87 79.24) (end 109.87 81.5425) (width 0.25) (layer "F.Cu") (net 18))
 (segment (start 108.5 73.9) (end 109 73.4) (width 0.25) (layer "F.Cu") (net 18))
 (segment (start 100.55 70.8) (end 100.55 76.6) (width 0.25) (layer "F.Cu") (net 18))
 (segment (start 107.39 72.9) (end 108.5 72.9) (width 0.25) (layer "F.Cu") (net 18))
 (segment (start 101.05 70.3) (end 100.55 70.8) (width 0.25) (layer "F.Cu") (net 18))
 (segment (start 101.51 76.9) (end 100.85 76.9) (width 0.25) (layer "F.Cu") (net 18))
 (segment (start 109.87 81.5425) (end 109.86 81.5525) (width 0.25) (layer "F.Cu") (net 18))
 (segment (start 107.39 75.4) (end 114.43 75.4) (width 0.25) (layer "F.Cu") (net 18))
 (segment (start 102.7 71.71) (end 102.7 70.95) (width 0.25) (layer "F.Cu") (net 18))
 (segment (start 108.5 72.9) (end 109 73.4) (width 0.25) (layer "F.Cu") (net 18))
 (segment (start 107.39 73.4) (end 109 73.4) (width 0.25) (layer "F.Cu") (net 18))
 (via (at 109 73.4) (size 0.8) (drill 0.4) (layers "F.Cu" "B.Cu") (free) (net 18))
 (via (at 109.85 77.5) (size 0.8) (drill 0.4) (layers "F.Cu" "B.Cu") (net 18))
 (via (at 103.35 70.3) (size 0.8) (drill 0.4) (layers "F.Cu" "B.Cu") (free) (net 18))
 (via (at 114.43 75.4) (size 0.8) (drill 0.4) (layers "F.Cu" "B.Cu") (free) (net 18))
 (via (at 107.1 70.3) (size 0.8) (drill 0.4) (layers "F.Cu" "B.Cu") (free) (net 18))
 (via (at 101.05 70.3) (size 0.8) (drill 0.4) (layers "F.Cu" "B.Cu") (free) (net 18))
 (segment (start 114.43 75.4) (end 109.87 75.4) (width 0.25) (layer "B.Cu") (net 18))
 (segment (start 109.85 77.5) (end 109.85 75.42) (width 0.25) (layer "B.Cu") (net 18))
 (segment (start 103.35 70.3) (end 101.05 70.3) (width 0.25) (layer "B.Cu") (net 18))
 (segment (start 109 73.4) (end 109 72.2) (width 0.25) (layer "B.Cu") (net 18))
 (segment (start 107.1 70.3) (end 103.35 70.3) (width 0.25) (layer "B.Cu") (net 18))
 (segment (start 109.55 73.95) (end 109 73.4) (width 0.25) (layer "B.Cu") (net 18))
 (segment (start 109.85 75.42) (end 109.85 73.95) (width 0.25) (layer "B.Cu") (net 18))
 (segment (start 109.85 73.95) (end 109.55 73.95) (width 0.25) (layer "B.Cu") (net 18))
 (segment (start 109 72.2) (end 107.1 70.3) (width 0.25) (layer "B.Cu") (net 18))
 (segment (start 109.87 75.4) (end 109.85 75.42) (width 0.25) (layer "B.Cu") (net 18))
 (segment (start 107.52 66.85) (end 107.52 64.14) (width 0.25) (layer "F.Cu") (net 11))
 (segment (start 106.2 68.57) (end 107.52 67.25) (width 0.25) (layer "F.Cu") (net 11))
 (segment (start 107.52 67.25) (end 107.52 66.85) (width 0.25) (layer "F.Cu") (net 11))
 (segment (start 106.2 71.71) (end 106.2 68.57) (width 0.25) (layer "F.Cu") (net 11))
 (segment (start 105.7 67.93) (end 105.02 67.25) (width 0.25) (layer "F.Cu") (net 8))
 (segment (start 105.7 71.71) (end 105.7 67.93) (width 0.25) (layer "F.Cu") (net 8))
 (segment (start 105.02 66.85) (end 105.02 64.18) (width 0.25) (layer "F.Cu") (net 8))
 (segment (start 105.02 67.25) (end 105.02 66.85) (width 0.25) (layer "F.Cu") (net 8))
 (segment (start 117.5 95.988) (end 117.5 94.05715) (width 0.25) (layer "F.Cu") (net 5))
 (segment (start 106.08 82.78) (end 104.55 81.25) (width 0.25) (layer "F.Cu") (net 12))
 (segment (start 107 96.92) (end 106.08 96) (width 0.25) (layer "F.Cu") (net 12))
 (segment (start 106.2 77.59) (end 106.2 79.8) (width 0.25) (layer "F.Cu") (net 12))
 (segment (start 106.08 96) (end 106.08 82.78) (width 0.25) (layer "F.Cu") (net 12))
 (segment (start 106.2 79.8) (end 106.55 80.15) (width 0.25) (layer "F.Cu") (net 12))
 (segment (start 104.55 81.25) (end 104.55 80.15) (width 0.25) (layer "F.Cu") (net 12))
 (via (at 104.55 80.15) (size 0.8) (drill 0.4) (layers "F.Cu" "B.Cu") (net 12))
 (via (at 106.55 80.15) (size 0.8) (drill 0.4) (layers "F.Cu" "B.Cu") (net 12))
 (segment (start 104.55 80.15) (end 106.55 80.15) (width 0.25) (layer "B.Cu") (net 12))
 (segment (start 105.7 81.3) (end 105.7 77.59) (width 0.25) (layer "F.Cu") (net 13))
 (segment (start 106.92 93.52) (end 106.92 82.49) (width 0.25) (layer "F.Cu") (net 13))
 (segment (start 109 95.6) (end 106.92 93.52) (width 0.25) (layer "F.Cu") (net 13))
 (segment (start 109 96.92) (end 109 95.6) (width 0.25) (layer "F.Cu") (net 13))
 (segment (start 106.92 82.49) (end 105.73 81.3) (width 0.25) (layer "F.Cu") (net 13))
 (segment (start 105.73 81.3) (end 105.7 81.3) (width 0.25) (layer "F.Cu") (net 13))
 (segment (start 105.2 69.53) (end 104.67 69) (width 0.25) (layer "F.Cu") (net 20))
 (segment (start 102.61 60.03) (end 108.775 60.03) (width 0.25) (layer "F.Cu") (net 20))
 (segment (start 105.2 71.71) (end 105.2 69.53) (width 0.25) (layer "F.Cu") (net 20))
 (segment (start 108.775 60.03) (end 109.91 58.895) (width 0.25) (layer "F.Cu") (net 20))
 (via (at 104.67 69) (size 0.8) (drill 0.4) (layers "F.Cu" "B.Cu") (free) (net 20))
 (via (at 102.61 60.03) (size 0.8) (drill 0.4) (layers "F.Cu" "B.Cu") (free) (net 20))
 (segment (start 104.67 69) (end 102.61 66.94) (width 0.25) (layer "B.Cu") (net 20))
 (segment (start 102.61 66.94) (end 102.61 60.03) (width 0.25) (layer "B.Cu") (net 20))
 (segment (start 109.99 60.78) (end 111.18 59.59) (width 0.25) (layer "F.Cu") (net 21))
 (segment (start 111.18 59.59) (end 111.18 58.895) (width 0.25) (layer "F.Cu") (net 21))
 (segment (start 104.7 71.71) (end 104.7 70.41) (width 0.25) (layer "F.Cu") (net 21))
 (segment (start 105.54 60.78) (end 109.99 60.78) (width 0.25) (layer "F.Cu") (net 21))
 (segment (start 103.47 69.18) (end 103.47 62.85) (width 0.25) (layer "F.Cu") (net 21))
 (segment (start 103.47 62.85) (end 105.54 60.78) (width 0.25) (layer "F.Cu") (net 21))
 (segment (start 104.7 70.41) (end 103.47 69.18) (width 0.25) (layer "F.Cu") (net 21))
 (segment (start 106.7 77.59) (end 106.7 78.86) (width 0.25) (layer "F.Cu") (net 24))
 (segment (start 111.17 53.48) (end 111.17 57.375) (width 0.25) (layer "F.Cu") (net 24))
 (segment (start 111.17 57.375) (end 111.18 57.375) (width 0.25) (layer "F.Cu") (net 24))
 (segment (start 108.01 84.98) (end 109.34 86.31) (width 0.25) (layer "F.Cu") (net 24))
 (segment (start 109.34 86.31) (end 109.85 86.31) (width 0.25) (layer "F.Cu") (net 24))
 (segment (start 106.7 78.86) (end 108.01 80.17) (width 0.25) (layer "F.Cu") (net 24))
 (segment (start 108.01 80.17) (end 108.01 84.98) (width 0.25) (layer "F.Cu") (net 24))
 (via (at 111.17 53.48) (size 0.8) (drill 0.4) (layers "F.Cu" "B.Cu") (free) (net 24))
 (via (at 109.85 86.31) (size 0.8) (drill 0.4) (layers "F.Cu" "B.Cu") (free) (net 24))
 (segment (start 115.41 80.75) (end 115.41 56.41) (width 0.25) (layer "B.Cu") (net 24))
 (segment (start 112.48 53.48) (end 111.17 53.48) (width 0.25) (layer "B.Cu") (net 24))
 (segment (start 109.85 86.31) (end 115.41 80.75) (width 0.25) (layer "B.Cu") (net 24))
 (segment (start 115.41 56.41) (end 112.48 53.48) (width 0.25) (layer "B.Cu") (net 24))
 (segment (start 109.288 72.4) (end 109.338 72.35) (width 0.25) (layer "F.Cu") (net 7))
 (segment (start 107.39 72.4) (end 109.288 72.4) (width 0.25) (layer "F.Cu") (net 7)))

